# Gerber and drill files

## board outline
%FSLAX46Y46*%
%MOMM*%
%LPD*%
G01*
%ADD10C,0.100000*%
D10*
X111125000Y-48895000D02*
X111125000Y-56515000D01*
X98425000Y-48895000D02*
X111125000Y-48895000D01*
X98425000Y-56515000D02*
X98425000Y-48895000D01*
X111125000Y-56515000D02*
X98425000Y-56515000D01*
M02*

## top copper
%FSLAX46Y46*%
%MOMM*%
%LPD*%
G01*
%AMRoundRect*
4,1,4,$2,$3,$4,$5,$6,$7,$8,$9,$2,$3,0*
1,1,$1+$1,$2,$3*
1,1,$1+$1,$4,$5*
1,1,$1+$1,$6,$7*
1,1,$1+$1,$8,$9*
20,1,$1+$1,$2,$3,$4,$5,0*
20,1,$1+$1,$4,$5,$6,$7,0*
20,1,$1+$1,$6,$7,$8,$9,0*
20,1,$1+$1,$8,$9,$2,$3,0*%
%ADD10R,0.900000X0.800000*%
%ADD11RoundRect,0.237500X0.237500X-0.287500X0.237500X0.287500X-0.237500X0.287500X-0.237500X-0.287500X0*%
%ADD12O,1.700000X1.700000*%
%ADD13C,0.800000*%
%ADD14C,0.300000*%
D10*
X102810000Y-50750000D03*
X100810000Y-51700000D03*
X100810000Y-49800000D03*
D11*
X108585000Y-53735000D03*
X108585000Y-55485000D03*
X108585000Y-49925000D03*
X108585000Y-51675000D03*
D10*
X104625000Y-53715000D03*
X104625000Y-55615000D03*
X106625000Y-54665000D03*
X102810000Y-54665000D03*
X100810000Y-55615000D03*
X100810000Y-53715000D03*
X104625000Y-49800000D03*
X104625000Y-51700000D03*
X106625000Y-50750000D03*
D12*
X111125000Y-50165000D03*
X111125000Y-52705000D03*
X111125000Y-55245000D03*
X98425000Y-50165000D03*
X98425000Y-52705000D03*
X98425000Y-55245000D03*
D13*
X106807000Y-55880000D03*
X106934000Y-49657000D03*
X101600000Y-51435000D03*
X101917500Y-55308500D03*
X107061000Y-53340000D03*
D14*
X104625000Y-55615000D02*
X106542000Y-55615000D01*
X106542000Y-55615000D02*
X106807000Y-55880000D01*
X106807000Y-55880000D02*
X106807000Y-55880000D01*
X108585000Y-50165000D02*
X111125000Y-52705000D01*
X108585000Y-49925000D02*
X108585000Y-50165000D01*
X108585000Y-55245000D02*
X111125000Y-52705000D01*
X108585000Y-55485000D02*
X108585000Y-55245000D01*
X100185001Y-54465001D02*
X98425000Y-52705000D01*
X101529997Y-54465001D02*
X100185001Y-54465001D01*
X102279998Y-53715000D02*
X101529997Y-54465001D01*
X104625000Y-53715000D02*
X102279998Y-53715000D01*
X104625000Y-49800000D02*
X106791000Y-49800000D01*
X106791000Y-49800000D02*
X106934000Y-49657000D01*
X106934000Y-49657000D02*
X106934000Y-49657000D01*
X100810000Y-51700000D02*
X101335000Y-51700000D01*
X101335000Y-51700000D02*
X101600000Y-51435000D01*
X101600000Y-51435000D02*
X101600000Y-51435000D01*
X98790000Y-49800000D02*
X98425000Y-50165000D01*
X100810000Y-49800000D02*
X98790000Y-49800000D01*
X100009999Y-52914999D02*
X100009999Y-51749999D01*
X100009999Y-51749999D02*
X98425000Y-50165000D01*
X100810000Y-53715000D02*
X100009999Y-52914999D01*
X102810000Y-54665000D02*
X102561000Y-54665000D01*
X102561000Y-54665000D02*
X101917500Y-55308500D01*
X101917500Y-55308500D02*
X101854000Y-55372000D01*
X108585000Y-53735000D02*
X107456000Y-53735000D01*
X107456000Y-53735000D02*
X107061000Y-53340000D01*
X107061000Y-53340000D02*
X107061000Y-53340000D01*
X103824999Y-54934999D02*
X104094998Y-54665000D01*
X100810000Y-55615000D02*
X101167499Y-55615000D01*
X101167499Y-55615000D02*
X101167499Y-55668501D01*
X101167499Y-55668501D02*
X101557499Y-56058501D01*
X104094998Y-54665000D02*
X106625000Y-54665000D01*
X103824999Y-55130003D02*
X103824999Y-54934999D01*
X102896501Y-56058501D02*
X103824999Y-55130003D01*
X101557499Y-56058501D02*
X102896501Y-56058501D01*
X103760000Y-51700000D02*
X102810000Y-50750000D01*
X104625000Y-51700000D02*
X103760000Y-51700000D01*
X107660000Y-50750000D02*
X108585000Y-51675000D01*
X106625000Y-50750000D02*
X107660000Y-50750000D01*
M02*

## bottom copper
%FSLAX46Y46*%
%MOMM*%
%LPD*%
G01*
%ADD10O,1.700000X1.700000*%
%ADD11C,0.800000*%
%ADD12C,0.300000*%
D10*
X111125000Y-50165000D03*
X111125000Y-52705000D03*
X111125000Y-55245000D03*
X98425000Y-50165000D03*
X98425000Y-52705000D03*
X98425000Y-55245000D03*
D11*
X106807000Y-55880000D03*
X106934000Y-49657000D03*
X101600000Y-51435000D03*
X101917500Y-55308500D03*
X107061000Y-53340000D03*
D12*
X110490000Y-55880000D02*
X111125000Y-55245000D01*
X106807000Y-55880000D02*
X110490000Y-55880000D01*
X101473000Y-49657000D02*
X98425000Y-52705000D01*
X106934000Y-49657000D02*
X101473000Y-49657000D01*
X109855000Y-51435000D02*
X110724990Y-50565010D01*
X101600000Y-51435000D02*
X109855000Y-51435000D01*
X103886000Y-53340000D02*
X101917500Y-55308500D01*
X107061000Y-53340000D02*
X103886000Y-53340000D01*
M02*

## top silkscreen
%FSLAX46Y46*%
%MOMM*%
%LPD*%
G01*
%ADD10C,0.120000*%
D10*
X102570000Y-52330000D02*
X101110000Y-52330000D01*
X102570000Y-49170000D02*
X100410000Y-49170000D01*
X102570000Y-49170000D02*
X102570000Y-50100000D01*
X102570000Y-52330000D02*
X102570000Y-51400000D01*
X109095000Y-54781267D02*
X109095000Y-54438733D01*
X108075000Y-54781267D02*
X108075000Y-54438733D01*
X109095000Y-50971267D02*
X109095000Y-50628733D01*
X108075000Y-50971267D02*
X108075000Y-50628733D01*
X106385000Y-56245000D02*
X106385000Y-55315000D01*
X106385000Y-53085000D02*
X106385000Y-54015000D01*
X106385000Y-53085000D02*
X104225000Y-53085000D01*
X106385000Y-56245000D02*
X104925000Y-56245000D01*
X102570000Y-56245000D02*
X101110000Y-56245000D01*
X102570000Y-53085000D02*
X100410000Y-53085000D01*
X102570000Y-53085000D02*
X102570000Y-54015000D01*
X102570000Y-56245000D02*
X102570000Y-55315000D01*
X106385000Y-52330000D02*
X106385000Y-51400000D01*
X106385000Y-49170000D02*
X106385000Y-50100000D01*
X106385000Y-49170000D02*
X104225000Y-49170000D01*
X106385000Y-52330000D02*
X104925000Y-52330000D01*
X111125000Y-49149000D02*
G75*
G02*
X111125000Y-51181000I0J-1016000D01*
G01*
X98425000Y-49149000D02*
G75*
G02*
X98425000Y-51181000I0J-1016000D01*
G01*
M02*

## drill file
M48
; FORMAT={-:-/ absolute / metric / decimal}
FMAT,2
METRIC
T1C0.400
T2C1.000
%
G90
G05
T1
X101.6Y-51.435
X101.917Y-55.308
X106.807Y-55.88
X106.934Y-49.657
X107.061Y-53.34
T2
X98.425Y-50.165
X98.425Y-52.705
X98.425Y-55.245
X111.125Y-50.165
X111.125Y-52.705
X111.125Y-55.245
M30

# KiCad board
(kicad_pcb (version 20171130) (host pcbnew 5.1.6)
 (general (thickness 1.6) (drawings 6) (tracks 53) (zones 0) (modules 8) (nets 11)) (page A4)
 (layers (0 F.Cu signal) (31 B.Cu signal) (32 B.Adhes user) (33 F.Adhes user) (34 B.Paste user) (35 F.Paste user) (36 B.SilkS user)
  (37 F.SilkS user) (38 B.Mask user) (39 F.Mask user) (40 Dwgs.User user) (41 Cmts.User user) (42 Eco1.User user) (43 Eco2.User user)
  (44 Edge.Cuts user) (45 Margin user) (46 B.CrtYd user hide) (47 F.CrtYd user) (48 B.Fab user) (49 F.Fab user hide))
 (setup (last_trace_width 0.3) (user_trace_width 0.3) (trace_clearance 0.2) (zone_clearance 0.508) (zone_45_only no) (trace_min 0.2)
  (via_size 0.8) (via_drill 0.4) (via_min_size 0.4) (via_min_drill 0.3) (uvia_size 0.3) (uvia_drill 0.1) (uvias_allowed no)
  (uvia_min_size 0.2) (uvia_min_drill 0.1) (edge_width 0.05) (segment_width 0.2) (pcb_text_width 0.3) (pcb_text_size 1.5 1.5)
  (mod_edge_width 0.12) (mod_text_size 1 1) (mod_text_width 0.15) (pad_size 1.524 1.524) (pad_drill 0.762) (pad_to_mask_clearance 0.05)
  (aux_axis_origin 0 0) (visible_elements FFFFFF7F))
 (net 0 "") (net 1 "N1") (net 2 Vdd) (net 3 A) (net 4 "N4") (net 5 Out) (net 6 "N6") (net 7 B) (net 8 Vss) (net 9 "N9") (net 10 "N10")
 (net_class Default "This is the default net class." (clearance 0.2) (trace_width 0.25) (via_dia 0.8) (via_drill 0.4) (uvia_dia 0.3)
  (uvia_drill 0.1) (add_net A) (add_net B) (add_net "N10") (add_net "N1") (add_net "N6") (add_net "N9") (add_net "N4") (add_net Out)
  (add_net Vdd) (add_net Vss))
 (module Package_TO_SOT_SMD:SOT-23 (layer F.Cu) (at 101.81 50.75)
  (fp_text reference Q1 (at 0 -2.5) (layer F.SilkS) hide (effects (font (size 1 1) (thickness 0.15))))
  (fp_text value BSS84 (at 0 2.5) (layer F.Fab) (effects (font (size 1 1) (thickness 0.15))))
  (fp_line (start 0.76 1.58) (end -0.7 1.58) (layer F.SilkS) (width 0.12))
  (fp_line (start 0.76 -1.58) (end -1.4 -1.58) (layer F.SilkS) (width 0.12))
  (fp_line (start 0.76 -1.58) (end 0.76 -0.65) (layer F.SilkS) (width 0.12))
  (fp_line (start 0.76 1.58) (end 0.76 0.65) (layer F.SilkS) (width 0.12))
  (pad 3 smd rect (at 1 0) (size 0.9 0.8) (layers F.Cu F.Paste F.Mask) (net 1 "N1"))
  (pad 2 smd rect (at -1 0.95) (size 0.9 0.8) (layers F.Cu F.Paste F.Mask) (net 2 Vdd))
  (pad 1 smd rect (at -1 -0.95) (size 0.9 0.8) (layers F.Cu F.Paste F.Mask) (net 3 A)))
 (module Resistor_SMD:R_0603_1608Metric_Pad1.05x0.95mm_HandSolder (layer F.Cu) (at 108.585 54.61 90)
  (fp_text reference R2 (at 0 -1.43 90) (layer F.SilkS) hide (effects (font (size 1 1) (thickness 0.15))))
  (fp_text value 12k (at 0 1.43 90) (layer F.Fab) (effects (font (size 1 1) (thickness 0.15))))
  (fp_line (start -0.171267 0.51) (end 0.171267 0.51) (layer F.SilkS) (width 0.12))
  (fp_line (start -0.171267 -0.51) (end 0.171267 -0.51) (layer F.SilkS) (width 0.12))
  (pad 2 smd roundrect (at 0.875 0 90) (size 1.05 0.95) (layers F.Cu F.Paste F.Mask) (roundrect_rratio 0.25) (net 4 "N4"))
  (pad 1 smd roundrect (at -0.875 0 90) (size 1.05 0.95) (layers F.Cu F.Paste F.Mask) (roundrect_rratio 0.25) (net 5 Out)))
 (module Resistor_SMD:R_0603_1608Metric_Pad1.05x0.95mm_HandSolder (layer F.Cu) (at 108.585 50.8 90)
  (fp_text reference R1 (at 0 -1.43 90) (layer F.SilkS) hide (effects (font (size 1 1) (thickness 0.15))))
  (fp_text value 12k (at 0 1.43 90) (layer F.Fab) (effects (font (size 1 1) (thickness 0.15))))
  (fp_line (start -0.171267 0.51) (end 0.171267 0.51) (layer F.SilkS) (width 0.12))
  (fp_line (start -0.171267 -0.51) (end 0.171267 -0.51) (layer F.SilkS) (width 0.12))
  (pad 2 smd roundrect (at 0.875 0 90) (size 1.05 0.95) (layers F.Cu F.Paste F.Mask) (roundrect_rratio 0.25) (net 5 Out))
  (pad 1 smd roundrect (at -0.875 0 90) (size 1.05 0.95) (layers F.Cu F.Paste F.Mask) (roundrect_rratio 0.25) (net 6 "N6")))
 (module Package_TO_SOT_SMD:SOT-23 (layer F.Cu) (at 105.625 54.665)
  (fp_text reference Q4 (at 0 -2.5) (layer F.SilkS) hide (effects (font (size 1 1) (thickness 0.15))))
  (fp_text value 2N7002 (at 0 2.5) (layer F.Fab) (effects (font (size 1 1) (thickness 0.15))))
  (fp_line (start 0.76 1.58) (end 0.76 0.65) (layer F.SilkS) (width 0.12))
  (fp_line (start 0.76 -1.58) (end 0.76 -0.65) (layer F.SilkS) (width 0.12))
  (fp_line (start 0.76 -1.58) (end -1.4 -1.58) (layer F.SilkS) (width 0.12))
  (fp_line (start 0.76 1.58) (end -0.7 1.58) (layer F.SilkS) (width 0.12))
  (pad 1 smd rect (at -1 -0.95) (size 0.9 0.8) (layers F.Cu F.Paste F.Mask) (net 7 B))
  (pad 2 smd rect (at -1 0.95) (size 0.9 0.8) (layers F.Cu F.Paste F.Mask) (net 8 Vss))
  (pad 3 smd rect (at 1 0) (size 0.9 0.8) (layers F.Cu F.Paste F.Mask) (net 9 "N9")))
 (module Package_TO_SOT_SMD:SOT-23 (layer F.Cu) (at 101.81 54.665)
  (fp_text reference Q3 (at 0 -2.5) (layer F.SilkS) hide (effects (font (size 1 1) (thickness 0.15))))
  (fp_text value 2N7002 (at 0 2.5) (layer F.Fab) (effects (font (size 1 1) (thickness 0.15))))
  (fp_line (start 0.76 1.58) (end -0.7 1.58) (layer F.SilkS) (width 0.12))
  (fp_line (start 0.76 -1.58) (end -1.4 -1.58) (layer F.SilkS) (width 0.12))
  (fp_line (start 0.76 -1.58) (end 0.76 -0.65) (layer F.SilkS) (width 0.12))
  (fp_line (start 0.76 1.58) (end 0.76 0.65) (layer F.SilkS) (width 0.12))
  (pad 3 smd rect (at 1 0) (size 0.9 0.8) (layers F.Cu F.Paste F.Mask) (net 4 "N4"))
  (pad 2 smd rect (at -1 0.95) (size 0.9 0.8) (layers F.Cu F.Paste F.Mask) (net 9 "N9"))
  (pad 1 smd rect (at -1 -0.95) (size 0.9 0.8) (layers F.Cu F.Paste F.Mask) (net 3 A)))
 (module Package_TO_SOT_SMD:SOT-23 (layer F.Cu) (at 105.625 50.75)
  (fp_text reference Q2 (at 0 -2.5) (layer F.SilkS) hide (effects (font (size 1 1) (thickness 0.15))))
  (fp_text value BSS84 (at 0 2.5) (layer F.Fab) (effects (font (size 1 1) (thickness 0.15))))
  (fp_line (start 0.76 1.58) (end 0.76 0.65) (layer F.SilkS) (width 0.12))
  (fp_line (start 0.76 -1.58) (end 0.76 -0.65) (layer F.SilkS) (width 0.12))
  (fp_line (start 0.76 -1.58) (end -1.4 -1.58) (layer F.SilkS) (width 0.12))
  (fp_line (start 0.76 1.58) (end -0.7 1.58) (layer F.SilkS) (width 0.12))
  (pad 1 smd rect (at -1 -0.95) (size 0.9 0.8) (layers F.Cu F.Paste F.Mask) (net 7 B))
  (pad 2 smd rect (at -1 0.95) (size 0.9 0.8) (layers F.Cu F.Paste F.Mask) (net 1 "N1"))
  (pad 3 smd rect (at 1 0) (size 0.9 0.8) (layers F.Cu F.Paste F.Mask) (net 6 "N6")))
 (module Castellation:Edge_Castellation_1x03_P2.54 (layer F.Cu) (at 111.125 50.165)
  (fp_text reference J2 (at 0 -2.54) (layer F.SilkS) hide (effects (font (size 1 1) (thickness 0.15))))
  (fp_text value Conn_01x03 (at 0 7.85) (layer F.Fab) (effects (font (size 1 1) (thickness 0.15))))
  (fp_arc (start 0 0) (end 0 1.016) (angle -180) (layer F.SilkS) (width 0.12))
  (pad 1 thru_hole oval (at 0 0) (size 1.7 1.7) (drill 1) (layers *.Cu *.Mask) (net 2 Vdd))
  (pad 2 thru_hole oval (at 0 2.54) (size 1.7 1.7) (drill 1) (layers *.Cu *.Mask) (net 5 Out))
  (pad 3 thru_hole oval (at 0 5.08) (size 1.7 1.7) (drill 1) (layers *.Cu *.Mask) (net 8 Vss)))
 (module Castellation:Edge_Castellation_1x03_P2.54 (layer F.Cu) (at 98.425 50.165)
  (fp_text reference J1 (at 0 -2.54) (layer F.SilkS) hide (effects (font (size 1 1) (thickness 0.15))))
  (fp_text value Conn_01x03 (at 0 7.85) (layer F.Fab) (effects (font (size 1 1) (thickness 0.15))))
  (fp_arc (start 0 0) (end 0 1.016) (angle -180) (layer F.SilkS) (width 0.12))
  (pad 1 thru_hole oval (at 0 0) (size 1.7 1.7) (drill 1) (layers *.Cu *.Mask) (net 3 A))
  (pad 2 thru_hole oval (at 0 2.54) (size 1.7 1.7) (drill 1) (layers *.Cu *.Mask) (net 7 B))
  (pad 3 thru_hole oval (at 0 5.08) (size 1.7 1.7) (drill 1) (layers *.Cu *.Mask) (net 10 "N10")))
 (gr_line (start 111.125 48.895) (end 111.125 56.515) (layer Edge.Cuts) (width 0.1))
 (gr_line (start 98.425 48.895) (end 111.125 48.895) (layer Edge.Cuts) (width 0.1))
 (gr_line (start 98.425 56.515) (end 98.425 48.895) (layer Edge.Cuts) (width 0.1))
 (gr_line (start 111.125 56.515) (end 98.425 56.515) (layer Edge.Cuts) (width 0.1))
 (segment (start 104.625 55.615) (end 106.542 55.615) (width 0.3) (layer F.Cu) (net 8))
 (segment (start 106.542 55.615) (end 106.807 55.88) (width 0.3) (layer F.Cu) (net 8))
 (segment (start 106.807 55.88) (end 106.807 55.88) (width 0.3) (layer F.Cu) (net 8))
 (via (at 106.807 55.88) (size 0.8) (drill 0.4) (layers F.Cu B.Cu) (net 8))
 (segment (start 110.49 55.88) (end 111.125 55.245) (width 0.3) (layer B.Cu) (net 8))
 (segment (start 106.807 55.88) (end 110.49 55.88) (width 0.3) (layer B.Cu) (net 8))
 (segment (start 108.585 50.165) (end 111.125 52.705) (width 0.3) (layer F.Cu) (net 5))
 (segment (start 108.585 49.925) (end 108.585 50.165) (width 0.3) (layer F.Cu) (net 5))
 (segment (start 108.585 55.245) (end 111.125 52.705) (width 0.3) (layer F.Cu) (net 5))
 (segment (start 108.585 55.485) (end 108.585 55.245) (width 0.3) (layer F.Cu) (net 5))
 (segment (start 100.185001 54.465001) (end 98.425 52.705) (width 0.3) (layer F.Cu) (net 7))
 (segment (start 101.529997 54.465001) (end 100.185001 54.465001) (width 0.3) (layer F.Cu) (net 7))
 (segment (start 102.279998 53.715) (end 101.529997 54.465001) (width 0.3) (layer F.Cu) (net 7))
 (segment (start 104.625 53.715) (end 102.279998 53.715) (width 0.3) (layer F.Cu) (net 7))
 (segment (start 104.625 49.8) (end 106.791 49.8) (width 0.3) (layer F.Cu) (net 7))
 (segment (start 106.791 49.8) (end 106.934 49.657) (width 0.3) (layer F.Cu) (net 7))
 (segment (start 106.934 49.657) (end 106.934 49.657) (width 0.3) (layer F.Cu) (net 7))
 (via (at 106.934 49.657) (size 0.8) (drill 0.4) (layers F.Cu B.Cu) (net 7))
 (segment (start 101.473 49.657) (end 98.425 52.705) (width 0.3) (layer B.Cu) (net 7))
 (segment (start 106.934 49.657) (end 101.473 49.657) (width 0.3) (layer B.Cu) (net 7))
 (segment (start 100.81 51.7) (end 101.335 51.7) (width 0.3) (layer F.Cu) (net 2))
 (segment (start 101.335 51.7) (end 101.6 51.435) (width 0.3) (layer F.Cu) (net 2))
 (segment (start 101.6 51.435) (end 101.6 51.435) (width 0.3) (layer F.Cu) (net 2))
 (via (at 101.6 51.435) (size 0.8) (drill 0.4) (layers F.Cu B.Cu) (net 2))
 (segment (start 109.855 51.435) (end 110.72499 50.56501) (width 0.3) (layer B.Cu) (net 2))
 (segment (start 101.6 51.435) (end 109.855 51.435) (width 0.3) (layer B.Cu) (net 2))
 (segment (start 98.79 49.8) (end 98.425 50.165) (width 0.3) (layer F.Cu) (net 3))
 (segment (start 100.81 49.8) (end 98.79 49.8) (width 0.3) (layer F.Cu) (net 3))
 (segment (start 100.009999 52.914999) (end 100.009999 51.749999) (width 0.3) (layer F.Cu) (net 3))
 (segment (start 100.009999 51.749999) (end 98.425 50.165) (width 0.3) (layer F.Cu) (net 3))
 (segment (start 100.81 53.715) (end 100.009999 52.914999) (width 0.3) (layer F.Cu) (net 3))
 (segment (start 102.81 54.665) (end 102.561 54.665) (width 0.3) (layer F.Cu) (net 4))
 (segment (start 102.561 54.665) (end 101.9175 55.3085) (width 0.3) (layer F.Cu) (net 4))
 (segment (start 101.9175 55.3085) (end 101.854 55.372) (width 0.3) (layer F.Cu) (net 4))
 (via (at 101.9175 55.3085) (size 0.8) (drill 0.4) (layers F.Cu B.Cu) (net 4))
 (segment (start 108.585 53.735) (end 107.456 53.735) (width 0.3) (layer F.Cu) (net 4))
 (segment (start 107.456 53.735) (end 107.061 53.34) (width 0.3) (layer F.Cu) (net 4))
 (segment (start 107.061 53.34) (end 107.061 53.34) (width 0.3) (layer F.Cu) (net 4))
 (via (at 107.061 53.34) (size 0.8) (drill 0.4) (layers F.Cu B.Cu) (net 4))
 (segment (start 103.886 53.34) (end 101.9175 55.3085) (width 0.3) (layer B.Cu) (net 4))
 (segment (start 107.061 53.34) (end 103.886 53.34) (width 0.3) (layer B.Cu) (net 4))
 (segment (start 103.824999 54.934999) (end 104.094998 54.665) (width 0.3) (layer F.Cu) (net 9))
 (segment (start 100.81 55.615) (end 101.167499 55.615) (width 0.3) (layer F.Cu) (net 9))
 (segment (start 101.167499 55.615) (end 101.167499 55.668501) (width 0.3) (layer F.Cu) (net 9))
 (segment (start 101.167499 55.668501) (end 101.557499 56.058501) (width 0.3) (layer F.Cu) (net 9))
 (segment (start 104.094998 54.665) (end 106.625 54.665) (width 0.3) (layer F.Cu) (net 9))
 (segment (start 103.824999 55.130003) (end 103.824999 54.934999) (width 0.3) (layer F.Cu) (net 9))
 (segment (start 102.896501 56.058501) (end 103.824999 55.130003) (width 0.3) (layer F.Cu) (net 9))
 (segment (start 101.557499 56.058501) (end 102.896501 56.058501) (width 0.3) (layer F.Cu) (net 9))
 (segment (start 103.76 51.7) (end 102.81 50.75) (width 0.3) (layer F.Cu) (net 1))
 (segment (start 104.625 51.7) (end 103.76 51.7) (width 0.3) (layer F.Cu) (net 1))
 (segment (start 107.66 50.75) (end 108.585 51.675) (width 0.3) (layer F.Cu) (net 6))
 (segment (start 106.625 50.75) (end 107.66 50.75) (width 0.3) (layer F.Cu) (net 6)))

